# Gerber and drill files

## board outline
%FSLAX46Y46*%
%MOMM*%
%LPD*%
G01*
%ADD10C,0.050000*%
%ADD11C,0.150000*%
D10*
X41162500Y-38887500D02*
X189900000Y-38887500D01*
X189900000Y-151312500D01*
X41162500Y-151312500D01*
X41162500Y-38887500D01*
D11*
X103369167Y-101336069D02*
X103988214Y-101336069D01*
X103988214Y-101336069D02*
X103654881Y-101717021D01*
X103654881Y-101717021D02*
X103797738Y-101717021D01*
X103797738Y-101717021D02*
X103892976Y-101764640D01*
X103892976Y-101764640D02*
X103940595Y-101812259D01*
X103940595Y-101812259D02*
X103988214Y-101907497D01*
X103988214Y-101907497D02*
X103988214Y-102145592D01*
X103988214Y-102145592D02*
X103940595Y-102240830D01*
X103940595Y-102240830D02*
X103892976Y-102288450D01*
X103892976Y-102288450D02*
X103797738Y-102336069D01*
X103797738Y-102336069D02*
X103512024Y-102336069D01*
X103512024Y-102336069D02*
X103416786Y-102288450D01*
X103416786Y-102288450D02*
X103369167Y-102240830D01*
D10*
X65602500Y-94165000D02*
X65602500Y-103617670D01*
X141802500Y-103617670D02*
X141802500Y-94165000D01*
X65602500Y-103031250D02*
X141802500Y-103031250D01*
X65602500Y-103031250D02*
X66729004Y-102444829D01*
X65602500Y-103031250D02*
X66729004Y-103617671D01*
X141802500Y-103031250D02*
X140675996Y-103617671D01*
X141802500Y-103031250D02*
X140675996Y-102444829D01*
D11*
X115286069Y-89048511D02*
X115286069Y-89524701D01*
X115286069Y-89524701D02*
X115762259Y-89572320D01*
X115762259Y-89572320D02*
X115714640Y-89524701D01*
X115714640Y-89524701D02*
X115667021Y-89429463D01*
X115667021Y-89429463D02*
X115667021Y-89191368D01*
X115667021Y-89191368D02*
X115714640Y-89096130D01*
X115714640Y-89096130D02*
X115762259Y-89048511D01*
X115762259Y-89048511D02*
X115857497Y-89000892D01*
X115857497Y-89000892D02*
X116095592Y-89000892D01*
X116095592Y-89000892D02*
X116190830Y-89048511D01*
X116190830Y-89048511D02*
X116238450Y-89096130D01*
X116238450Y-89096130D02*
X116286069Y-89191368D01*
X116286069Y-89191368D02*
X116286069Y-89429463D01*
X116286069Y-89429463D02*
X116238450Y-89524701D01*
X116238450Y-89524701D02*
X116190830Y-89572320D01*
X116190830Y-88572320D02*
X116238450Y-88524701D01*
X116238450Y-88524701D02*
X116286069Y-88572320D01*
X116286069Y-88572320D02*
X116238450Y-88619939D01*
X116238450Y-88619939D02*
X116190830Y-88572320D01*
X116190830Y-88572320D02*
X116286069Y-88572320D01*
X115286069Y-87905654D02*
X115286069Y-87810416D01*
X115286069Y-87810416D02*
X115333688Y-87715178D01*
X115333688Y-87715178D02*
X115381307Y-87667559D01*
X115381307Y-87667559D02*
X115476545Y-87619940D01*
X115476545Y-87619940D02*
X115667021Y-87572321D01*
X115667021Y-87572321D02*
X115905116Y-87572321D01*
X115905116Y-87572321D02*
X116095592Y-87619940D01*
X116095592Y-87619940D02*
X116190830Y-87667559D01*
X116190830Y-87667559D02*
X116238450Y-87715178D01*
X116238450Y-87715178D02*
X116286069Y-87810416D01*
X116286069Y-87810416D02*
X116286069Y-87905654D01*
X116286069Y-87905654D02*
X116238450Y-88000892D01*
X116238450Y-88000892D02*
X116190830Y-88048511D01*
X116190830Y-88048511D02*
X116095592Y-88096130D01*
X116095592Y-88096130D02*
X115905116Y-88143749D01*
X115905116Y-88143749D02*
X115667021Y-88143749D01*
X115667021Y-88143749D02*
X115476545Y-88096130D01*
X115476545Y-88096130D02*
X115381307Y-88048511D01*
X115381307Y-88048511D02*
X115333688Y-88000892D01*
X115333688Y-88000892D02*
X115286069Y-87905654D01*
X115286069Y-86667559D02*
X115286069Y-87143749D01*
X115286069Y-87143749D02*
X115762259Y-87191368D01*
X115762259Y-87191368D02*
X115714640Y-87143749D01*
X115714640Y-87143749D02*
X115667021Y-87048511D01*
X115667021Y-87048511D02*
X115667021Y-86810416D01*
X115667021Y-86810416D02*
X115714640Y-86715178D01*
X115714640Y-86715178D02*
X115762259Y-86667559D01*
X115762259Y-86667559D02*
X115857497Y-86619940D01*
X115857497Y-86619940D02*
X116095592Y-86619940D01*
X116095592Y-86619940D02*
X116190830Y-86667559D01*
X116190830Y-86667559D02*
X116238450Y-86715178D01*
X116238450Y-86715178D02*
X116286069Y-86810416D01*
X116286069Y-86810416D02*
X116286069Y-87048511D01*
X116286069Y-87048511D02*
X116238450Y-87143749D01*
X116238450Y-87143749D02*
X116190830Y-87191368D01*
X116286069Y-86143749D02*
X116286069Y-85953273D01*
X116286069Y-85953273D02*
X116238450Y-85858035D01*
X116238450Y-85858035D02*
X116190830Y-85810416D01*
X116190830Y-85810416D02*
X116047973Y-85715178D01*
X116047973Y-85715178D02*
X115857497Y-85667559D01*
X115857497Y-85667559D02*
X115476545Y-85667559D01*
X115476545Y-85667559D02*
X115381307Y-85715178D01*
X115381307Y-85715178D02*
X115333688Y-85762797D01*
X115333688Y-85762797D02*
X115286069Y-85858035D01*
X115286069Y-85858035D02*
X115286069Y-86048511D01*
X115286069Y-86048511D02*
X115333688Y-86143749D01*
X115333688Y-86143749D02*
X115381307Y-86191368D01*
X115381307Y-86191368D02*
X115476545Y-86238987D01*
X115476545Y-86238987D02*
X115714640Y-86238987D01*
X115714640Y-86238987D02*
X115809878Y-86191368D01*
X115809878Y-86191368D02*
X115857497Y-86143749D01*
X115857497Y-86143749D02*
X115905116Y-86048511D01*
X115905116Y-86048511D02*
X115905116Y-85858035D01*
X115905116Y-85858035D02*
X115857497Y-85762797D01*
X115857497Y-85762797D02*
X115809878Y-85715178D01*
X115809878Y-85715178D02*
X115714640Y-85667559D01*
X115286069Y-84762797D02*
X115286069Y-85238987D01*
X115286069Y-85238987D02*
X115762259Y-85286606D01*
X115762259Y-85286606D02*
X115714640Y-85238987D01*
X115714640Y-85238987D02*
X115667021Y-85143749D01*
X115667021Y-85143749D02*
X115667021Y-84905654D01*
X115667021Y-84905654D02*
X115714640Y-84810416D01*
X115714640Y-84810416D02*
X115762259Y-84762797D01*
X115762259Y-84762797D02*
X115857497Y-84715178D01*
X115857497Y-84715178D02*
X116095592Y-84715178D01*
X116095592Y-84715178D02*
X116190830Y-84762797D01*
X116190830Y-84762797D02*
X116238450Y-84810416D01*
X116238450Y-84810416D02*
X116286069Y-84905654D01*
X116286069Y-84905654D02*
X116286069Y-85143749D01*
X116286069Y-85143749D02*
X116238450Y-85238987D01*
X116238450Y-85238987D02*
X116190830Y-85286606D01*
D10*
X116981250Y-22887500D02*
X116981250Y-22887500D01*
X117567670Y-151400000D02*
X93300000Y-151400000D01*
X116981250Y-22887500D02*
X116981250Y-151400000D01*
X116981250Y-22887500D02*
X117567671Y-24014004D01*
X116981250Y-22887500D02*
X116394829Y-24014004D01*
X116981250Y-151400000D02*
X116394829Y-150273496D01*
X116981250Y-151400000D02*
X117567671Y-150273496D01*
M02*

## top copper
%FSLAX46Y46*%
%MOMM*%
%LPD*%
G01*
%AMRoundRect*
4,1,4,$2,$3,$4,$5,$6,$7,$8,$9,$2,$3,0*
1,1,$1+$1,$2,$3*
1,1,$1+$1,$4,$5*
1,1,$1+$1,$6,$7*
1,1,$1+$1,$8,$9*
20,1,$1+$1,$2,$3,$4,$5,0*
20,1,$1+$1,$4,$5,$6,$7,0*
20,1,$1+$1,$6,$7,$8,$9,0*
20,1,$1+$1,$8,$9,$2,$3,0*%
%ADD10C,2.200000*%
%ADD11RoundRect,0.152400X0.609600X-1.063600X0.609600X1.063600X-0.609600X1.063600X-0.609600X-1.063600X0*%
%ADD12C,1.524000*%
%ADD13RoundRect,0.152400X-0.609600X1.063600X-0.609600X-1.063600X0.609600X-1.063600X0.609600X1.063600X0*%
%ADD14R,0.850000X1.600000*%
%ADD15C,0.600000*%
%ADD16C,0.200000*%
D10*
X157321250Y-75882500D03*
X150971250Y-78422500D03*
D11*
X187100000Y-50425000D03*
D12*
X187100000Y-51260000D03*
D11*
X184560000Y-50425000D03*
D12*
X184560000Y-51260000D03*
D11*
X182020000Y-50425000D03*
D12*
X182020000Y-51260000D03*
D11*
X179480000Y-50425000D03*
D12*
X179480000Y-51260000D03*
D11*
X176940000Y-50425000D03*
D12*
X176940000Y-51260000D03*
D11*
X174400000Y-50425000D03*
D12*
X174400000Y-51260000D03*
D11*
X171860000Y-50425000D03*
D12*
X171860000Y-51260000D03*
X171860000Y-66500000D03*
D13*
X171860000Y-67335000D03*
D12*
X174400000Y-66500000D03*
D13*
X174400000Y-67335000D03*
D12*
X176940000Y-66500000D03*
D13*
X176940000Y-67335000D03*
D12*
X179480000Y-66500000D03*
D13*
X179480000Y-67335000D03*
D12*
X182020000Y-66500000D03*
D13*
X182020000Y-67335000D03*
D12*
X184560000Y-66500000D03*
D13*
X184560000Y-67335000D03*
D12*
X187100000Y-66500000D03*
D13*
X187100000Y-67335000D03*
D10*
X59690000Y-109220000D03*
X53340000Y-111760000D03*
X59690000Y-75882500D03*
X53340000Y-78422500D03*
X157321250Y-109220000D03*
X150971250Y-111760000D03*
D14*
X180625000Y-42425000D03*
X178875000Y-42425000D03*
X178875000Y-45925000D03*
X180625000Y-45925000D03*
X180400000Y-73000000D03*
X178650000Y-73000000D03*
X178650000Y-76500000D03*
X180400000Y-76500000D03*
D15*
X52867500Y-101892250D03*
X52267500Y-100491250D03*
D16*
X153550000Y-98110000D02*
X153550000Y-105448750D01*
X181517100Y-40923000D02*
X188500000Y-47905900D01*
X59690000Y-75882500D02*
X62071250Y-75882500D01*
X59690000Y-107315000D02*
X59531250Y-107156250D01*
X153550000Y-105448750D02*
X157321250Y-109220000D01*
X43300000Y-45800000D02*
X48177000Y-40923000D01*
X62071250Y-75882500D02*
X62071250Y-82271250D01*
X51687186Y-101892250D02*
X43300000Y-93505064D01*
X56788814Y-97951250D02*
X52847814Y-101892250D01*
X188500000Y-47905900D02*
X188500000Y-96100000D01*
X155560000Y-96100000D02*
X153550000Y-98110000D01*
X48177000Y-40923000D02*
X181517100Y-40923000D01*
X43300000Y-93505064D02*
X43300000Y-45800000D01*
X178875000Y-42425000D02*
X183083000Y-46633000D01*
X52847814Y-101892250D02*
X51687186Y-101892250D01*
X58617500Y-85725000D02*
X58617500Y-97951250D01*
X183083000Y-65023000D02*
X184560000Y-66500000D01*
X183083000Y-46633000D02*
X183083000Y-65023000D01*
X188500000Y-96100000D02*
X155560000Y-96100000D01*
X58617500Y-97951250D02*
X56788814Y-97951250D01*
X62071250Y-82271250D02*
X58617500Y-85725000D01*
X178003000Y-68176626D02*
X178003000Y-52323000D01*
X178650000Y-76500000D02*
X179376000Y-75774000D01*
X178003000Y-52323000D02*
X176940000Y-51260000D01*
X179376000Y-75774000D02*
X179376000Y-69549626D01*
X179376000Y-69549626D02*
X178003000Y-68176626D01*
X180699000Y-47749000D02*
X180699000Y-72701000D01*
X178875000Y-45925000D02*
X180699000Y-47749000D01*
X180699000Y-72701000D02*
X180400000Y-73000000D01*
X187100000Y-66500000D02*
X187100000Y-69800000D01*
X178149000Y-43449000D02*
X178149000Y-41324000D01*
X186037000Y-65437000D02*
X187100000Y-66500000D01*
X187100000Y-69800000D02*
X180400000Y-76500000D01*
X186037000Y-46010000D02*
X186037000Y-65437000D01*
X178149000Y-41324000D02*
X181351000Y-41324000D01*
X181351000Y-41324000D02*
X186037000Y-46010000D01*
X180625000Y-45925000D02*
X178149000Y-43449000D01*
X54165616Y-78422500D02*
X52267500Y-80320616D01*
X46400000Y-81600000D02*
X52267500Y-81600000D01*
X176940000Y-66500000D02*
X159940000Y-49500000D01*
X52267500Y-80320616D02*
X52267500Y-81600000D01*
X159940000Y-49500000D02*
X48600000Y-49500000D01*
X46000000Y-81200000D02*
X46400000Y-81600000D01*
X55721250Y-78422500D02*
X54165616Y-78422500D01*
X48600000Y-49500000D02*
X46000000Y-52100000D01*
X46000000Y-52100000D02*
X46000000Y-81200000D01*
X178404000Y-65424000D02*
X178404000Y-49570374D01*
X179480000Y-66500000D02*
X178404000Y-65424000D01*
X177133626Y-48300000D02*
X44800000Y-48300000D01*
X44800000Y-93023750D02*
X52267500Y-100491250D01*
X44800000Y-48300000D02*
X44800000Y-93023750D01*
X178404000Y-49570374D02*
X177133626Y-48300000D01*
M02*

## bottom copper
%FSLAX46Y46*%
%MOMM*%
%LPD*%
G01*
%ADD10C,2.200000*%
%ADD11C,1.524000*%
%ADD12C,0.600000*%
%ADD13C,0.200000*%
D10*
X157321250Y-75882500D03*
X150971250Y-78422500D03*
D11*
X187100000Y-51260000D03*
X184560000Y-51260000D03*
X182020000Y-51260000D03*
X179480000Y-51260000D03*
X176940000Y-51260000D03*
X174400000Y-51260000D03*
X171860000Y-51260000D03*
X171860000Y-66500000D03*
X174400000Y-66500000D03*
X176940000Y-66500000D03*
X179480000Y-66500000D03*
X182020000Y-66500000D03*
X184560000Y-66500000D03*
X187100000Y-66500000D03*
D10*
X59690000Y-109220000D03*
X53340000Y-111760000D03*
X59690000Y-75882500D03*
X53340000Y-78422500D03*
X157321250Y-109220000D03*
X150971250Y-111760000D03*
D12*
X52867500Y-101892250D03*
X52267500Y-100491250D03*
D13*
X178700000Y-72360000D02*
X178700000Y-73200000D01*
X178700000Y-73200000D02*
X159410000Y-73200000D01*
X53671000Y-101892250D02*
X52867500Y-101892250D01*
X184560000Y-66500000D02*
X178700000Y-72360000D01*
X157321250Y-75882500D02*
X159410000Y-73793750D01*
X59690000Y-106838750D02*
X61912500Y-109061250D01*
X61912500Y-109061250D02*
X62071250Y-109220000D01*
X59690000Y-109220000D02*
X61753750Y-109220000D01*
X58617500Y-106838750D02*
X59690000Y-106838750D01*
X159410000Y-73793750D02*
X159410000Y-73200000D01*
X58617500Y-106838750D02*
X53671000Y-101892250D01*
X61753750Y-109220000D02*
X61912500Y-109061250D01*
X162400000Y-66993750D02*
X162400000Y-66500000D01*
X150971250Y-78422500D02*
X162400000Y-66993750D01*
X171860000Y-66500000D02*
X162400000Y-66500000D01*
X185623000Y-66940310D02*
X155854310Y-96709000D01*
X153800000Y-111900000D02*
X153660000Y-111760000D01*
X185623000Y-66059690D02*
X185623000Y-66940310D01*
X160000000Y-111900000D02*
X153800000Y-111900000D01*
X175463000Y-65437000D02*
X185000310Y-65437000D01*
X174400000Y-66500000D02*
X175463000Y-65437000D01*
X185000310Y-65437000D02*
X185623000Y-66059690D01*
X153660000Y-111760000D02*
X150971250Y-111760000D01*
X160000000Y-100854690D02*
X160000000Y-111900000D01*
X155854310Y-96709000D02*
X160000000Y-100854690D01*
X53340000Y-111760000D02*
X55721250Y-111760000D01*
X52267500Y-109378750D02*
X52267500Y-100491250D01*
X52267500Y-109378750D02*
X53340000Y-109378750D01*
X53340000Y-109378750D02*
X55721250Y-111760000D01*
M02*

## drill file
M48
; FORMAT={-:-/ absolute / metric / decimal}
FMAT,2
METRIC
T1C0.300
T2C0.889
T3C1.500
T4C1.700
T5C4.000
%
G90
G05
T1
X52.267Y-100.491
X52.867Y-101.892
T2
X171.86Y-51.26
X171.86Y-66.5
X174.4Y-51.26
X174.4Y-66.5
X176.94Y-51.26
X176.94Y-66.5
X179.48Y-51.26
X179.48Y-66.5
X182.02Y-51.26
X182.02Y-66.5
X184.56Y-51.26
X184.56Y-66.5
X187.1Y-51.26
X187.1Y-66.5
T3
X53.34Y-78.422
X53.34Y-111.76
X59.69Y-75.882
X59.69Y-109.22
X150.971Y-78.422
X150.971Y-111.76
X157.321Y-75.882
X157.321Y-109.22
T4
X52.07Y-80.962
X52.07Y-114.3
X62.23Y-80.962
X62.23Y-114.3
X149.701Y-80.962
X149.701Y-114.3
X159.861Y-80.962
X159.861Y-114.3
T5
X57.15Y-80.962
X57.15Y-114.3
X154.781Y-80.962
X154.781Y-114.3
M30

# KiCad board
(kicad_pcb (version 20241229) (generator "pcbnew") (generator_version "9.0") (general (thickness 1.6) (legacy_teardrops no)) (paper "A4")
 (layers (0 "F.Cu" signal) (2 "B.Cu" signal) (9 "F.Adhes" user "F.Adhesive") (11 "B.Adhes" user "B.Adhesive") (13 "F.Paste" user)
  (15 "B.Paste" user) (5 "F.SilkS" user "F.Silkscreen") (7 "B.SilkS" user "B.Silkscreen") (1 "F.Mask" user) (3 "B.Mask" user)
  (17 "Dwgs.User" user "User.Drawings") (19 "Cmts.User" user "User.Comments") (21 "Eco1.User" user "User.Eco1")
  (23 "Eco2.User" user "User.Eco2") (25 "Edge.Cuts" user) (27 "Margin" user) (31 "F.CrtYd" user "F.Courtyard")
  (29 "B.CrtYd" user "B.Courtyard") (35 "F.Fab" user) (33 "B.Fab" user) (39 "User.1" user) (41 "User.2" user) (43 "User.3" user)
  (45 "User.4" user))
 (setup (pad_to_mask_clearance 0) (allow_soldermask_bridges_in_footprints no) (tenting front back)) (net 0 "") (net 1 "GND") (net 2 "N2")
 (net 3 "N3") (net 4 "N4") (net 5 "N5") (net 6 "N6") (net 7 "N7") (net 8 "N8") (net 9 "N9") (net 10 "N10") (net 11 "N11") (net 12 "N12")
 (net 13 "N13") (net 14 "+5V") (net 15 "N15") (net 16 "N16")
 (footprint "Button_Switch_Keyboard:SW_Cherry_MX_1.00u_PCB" (layer "F.Cu") (at 157.32125 75.8825)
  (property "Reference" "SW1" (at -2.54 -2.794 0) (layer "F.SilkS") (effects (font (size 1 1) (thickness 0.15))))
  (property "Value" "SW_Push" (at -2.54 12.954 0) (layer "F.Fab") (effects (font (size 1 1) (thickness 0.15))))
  (pad "" np_thru_hole circle (at -7.62 5.08) (size 1.7 1.7) (drill 1.7) (layers "*.Cu" "*.Mask"))
  (pad "" np_thru_hole circle (at -2.54 5.08) (size 4 4) (drill 4) (layers "*.Cu" "*.Mask"))
  (pad "" np_thru_hole circle (at 2.54 5.08) (size 1.7 1.7) (drill 1.7) (layers "*.Cu" "*.Mask"))
  (pad "1" thru_hole circle (at 0 0) (size 2.2 2.2) (drill 1.5) (layers "*.Cu" "*.Mask") (remove_unused_layers no) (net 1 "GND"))
  (pad "2" thru_hole circle (at -6.35 2.54) (size 2.2 2.2) (drill 1.5) (layers "*.Cu" "*.Mask") (remove_unused_layers no) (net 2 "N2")))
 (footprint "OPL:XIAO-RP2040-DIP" (layer "F.Cu") (at 179.48 58.88 -90)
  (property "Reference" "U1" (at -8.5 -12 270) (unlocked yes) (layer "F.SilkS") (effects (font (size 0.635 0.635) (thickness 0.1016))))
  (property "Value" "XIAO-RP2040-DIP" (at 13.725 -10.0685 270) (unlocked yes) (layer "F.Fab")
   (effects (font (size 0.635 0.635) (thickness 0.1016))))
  (pad "1" smd roundrect (at -8.455 -7.62 90) (size 2.432 1.524) (layers "F.Cu" "F.Mask") (roundrect_rratio 0.1) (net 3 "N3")
   (thermal_bridge_angle 45))
  (pad "1" thru_hole circle (at -7.62 -7.62 90) (size 1.524 1.524) (drill 0.889) (layers "*.Cu" "*.Mask") (remove_unused_layers no)
   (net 3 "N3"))
  (pad "2" smd roundrect (at -8.455 -5.08 90) (size 2.432 1.524) (layers "F.Cu" "F.Mask") (roundrect_rratio 0.1) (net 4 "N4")
   (thermal_bridge_angle 45))
  (pad "2" thru_hole circle (at -7.62 -5.08 90) (size 1.524 1.524) (drill 0.889) (layers "*.Cu" "*.Mask") (remove_unused_layers no)
   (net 4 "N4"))
  (pad "3" smd roundrect (at -8.455 -2.54 90) (size 2.432 1.524) (layers "F.Cu" "F.Mask") (roundrect_rratio 0.1) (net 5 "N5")
   (thermal_bridge_angle 45))
  (pad "3" thru_hole circle (at -7.62 -2.54 90) (size 1.524 1.524) (drill 0.889) (layers "*.Cu" "*.Mask") (remove_unused_layers no)
   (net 5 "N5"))
  (pad "4" smd roundrect (at -8.455 0 90) (size 2.432 1.524) (layers "F.Cu" "F.Mask") (roundrect_rratio 0.1) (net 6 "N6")
   (thermal_bridge_angle 45))
  (pad "4" thru_hole circle (at -7.62 0 90) (size 1.524 1.524) (drill 0.889) (layers "*.Cu" "*.Mask") (remove_unused_layers no) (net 6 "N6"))
  (pad "5" smd roundrect (at -8.455 2.54 90) (size 2.432 1.524) (layers "F.Cu" "F.Mask") (roundrect_rratio 0.1) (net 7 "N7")
   (thermal_bridge_angle 45))
  (pad "5" thru_hole circle (at -7.62 2.54 90) (size 1.524 1.524) (drill 0.889) (layers "*.Cu" "*.Mask") (remove_unused_layers no)
   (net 7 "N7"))
  (pad "6" smd roundrect (at -8.455 5.08 90) (size 2.432 1.524) (layers "F.Cu" "F.Mask") (roundrect_rratio 0.1) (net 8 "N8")
   (thermal_bridge_angle 45))
  (pad "6" thru_hole circle (at -7.62 5.08 90) (size 1.524 1.524) (drill 0.889) (layers "*.Cu" "*.Mask") (remove_unused_layers no)
   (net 8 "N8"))
  (pad "7" smd roundrect (at -8.455 7.62 90) (size 2.432 1.524) (layers "F.Cu" "F.Mask") (roundrect_rratio 0.1) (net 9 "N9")
   (thermal_bridge_angle 45))
  (pad "7" thru_hole circle (at -7.62 7.62 90) (size 1.524 1.524) (drill 0.889) (layers "*.Cu" "*.Mask") (remove_unused_layers no)
   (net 9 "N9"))
  (pad "8" thru_hole circle (at 7.62 7.62 270) (size 1.524 1.524) (drill 0.889) (layers "*.Cu" "*.Mask") (remove_unused_layers no)
   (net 2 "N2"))
  (pad "8" smd roundrect (at 8.455 7.62 270) (size 2.432 1.524) (layers "F.Cu" "F.Mask") (roundrect_rratio 0.1) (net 2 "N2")
   (thermal_bridge_angle 45))
  (pad "9" thru_hole circle (at 7.62 5.08 270) (size 1.524 1.524) (drill 0.889) (layers "*.Cu" "*.Mask") (remove_unused_layers no)
   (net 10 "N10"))
  (pad "9" smd roundrect (at 8.455 5.08 270) (size 2.432 1.524) (layers "F.Cu" "F.Mask") (roundrect_rratio 0.1) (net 10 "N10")
   (thermal_bridge_angle 45))
  (pad "10" thru_hole circle (at 7.62 2.54 270) (size 1.524 1.524) (drill 0.889) (layers "*.Cu" "*.Mask") (remove_unused_layers no)
   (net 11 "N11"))
  (pad "10" smd roundrect (at 8.455 2.54 270) (size 2.432 1.524) (layers "F.Cu" "F.Mask") (roundrect_rratio 0.1) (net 11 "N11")
   (thermal_bridge_angle 45))
  (pad "11" thru_hole circle (at 7.62 0 270) (size 1.524 1.524) (drill 0.889) (layers "*.Cu" "*.Mask") (remove_unused_layers no)
   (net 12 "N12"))
  (pad "11" smd roundrect (at 8.455 0 270) (size 2.432 1.524) (layers "F.Cu" "F.Mask") (roundrect_rratio 0.1) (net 12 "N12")
   (thermal_bridge_angle 45))
  (pad "12" thru_hole circle (at 7.62 -2.54 270) (size 1.524 1.524) (drill 0.889) (layers "*.Cu" "*.Mask") (remove_unused_layers no)
   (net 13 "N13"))
  (pad "12" smd roundrect (at 8.455 -2.54 270) (size 2.432 1.524) (layers "F.Cu" "F.Mask") (roundrect_rratio 0.1) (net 13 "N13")
   (thermal_bridge_angle 45))
  (pad "13" thru_hole circle (at 7.62 -5.08 270) (size 1.524 1.524) (drill 0.889) (layers "*.Cu" "*.Mask") (remove_unused_layers no)
   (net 1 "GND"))
  (pad "13" smd roundrect (at 8.455 -5.08 270) (size 2.432 1.524) (layers "F.Cu" "F.Mask") (roundrect_rratio 0.1) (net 1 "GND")
   (thermal_bridge_angle 45))
  (pad "14" thru_hole circle (at 7.62 -7.62 270) (size 1.524 1.524) (drill 0.889) (layers "*.Cu" "*.Mask") (remove_unused_layers no)
   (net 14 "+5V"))
  (pad "14" smd roundrect (at 8.455 -7.62 270) (size 2.432 1.524) (layers "F.Cu" "F.Mask") (roundrect_rratio 0.1) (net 14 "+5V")
   (thermal_bridge_angle 45)))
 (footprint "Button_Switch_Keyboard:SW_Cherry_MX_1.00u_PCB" (layer "F.Cu") (at 59.69 109.22)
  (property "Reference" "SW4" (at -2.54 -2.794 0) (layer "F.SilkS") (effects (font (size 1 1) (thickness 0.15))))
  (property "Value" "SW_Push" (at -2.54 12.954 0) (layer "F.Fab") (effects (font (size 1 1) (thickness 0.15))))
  (pad "" np_thru_hole circle (at -7.62 5.08) (size 1.7 1.7) (drill 1.7) (layers "*.Cu" "*.Mask"))
  (pad "" np_thru_hole circle (at -2.54 5.08) (size 4 4) (drill 4) (layers "*.Cu" "*.Mask"))
  (pad "" np_thru_hole circle (at 2.54 5.08) (size 1.7 1.7) (drill 1.7) (layers "*.Cu" "*.Mask"))
  (pad "1" thru_hole circle (at 0 0) (size 2.2 2.2) (drill 1.5) (layers "*.Cu" "*.Mask") (remove_unused_layers no) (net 1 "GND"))
  (pad "2" thru_hole circle (at -6.35 2.54) (size 2.2 2.2) (drill 1.5) (layers "*.Cu" "*.Mask") (remove_unused_layers no) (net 12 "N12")))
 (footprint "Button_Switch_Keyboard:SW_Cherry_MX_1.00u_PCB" (layer "F.Cu") (at 59.69 75.8825)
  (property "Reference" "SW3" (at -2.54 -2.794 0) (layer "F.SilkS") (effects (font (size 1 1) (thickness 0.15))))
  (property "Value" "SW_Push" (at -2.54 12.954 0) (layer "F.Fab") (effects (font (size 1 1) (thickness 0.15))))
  (pad "" np_thru_hole circle (at -7.62 5.08) (size 1.7 1.7) (drill 1.7) (layers "*.Cu" "*.Mask"))
  (pad "" np_thru_hole circle (at -2.54 5.08) (size 4 4) (drill 4) (layers "*.Cu" "*.Mask"))
  (pad "" np_thru_hole circle (at 2.54 5.08) (size 1.7 1.7) (drill 1.7) (layers "*.Cu" "*.Mask"))
  (pad "1" thru_hole circle (at 0 0) (size 2.2 2.2) (drill 1.5) (layers "*.Cu" "*.Mask") (remove_unused_layers no) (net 1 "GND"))
  (pad "2" thru_hole circle (at -6.35 2.54) (size 2.2 2.2) (drill 1.5) (layers "*.Cu" "*.Mask") (remove_unused_layers no) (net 11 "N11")))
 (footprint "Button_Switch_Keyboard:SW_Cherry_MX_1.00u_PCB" (layer "F.Cu") (at 157.32125 109.22)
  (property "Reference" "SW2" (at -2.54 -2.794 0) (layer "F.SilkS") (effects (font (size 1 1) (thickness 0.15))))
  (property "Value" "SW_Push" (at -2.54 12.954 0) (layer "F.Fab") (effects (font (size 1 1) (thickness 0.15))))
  (pad "" np_thru_hole circle (at -7.62 5.08) (size 1.7 1.7) (drill 1.7) (layers "*.Cu" "*.Mask"))
  (pad "" np_thru_hole circle (at -2.54 5.08) (size 4 4) (drill 4) (layers "*.Cu" "*.Mask"))
  (pad "" np_thru_hole circle (at 2.54 5.08) (size 1.7 1.7) (drill 1.7) (layers "*.Cu" "*.Mask"))
  (pad "1" thru_hole circle (at 0 0) (size 2.2 2.2) (drill 1.5) (layers "*.Cu" "*.Mask") (remove_unused_layers no) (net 1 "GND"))
  (pad "2" thru_hole circle (at -6.35 2.54) (size 2.2 2.2) (drill 1.5) (layers "*.Cu" "*.Mask") (remove_unused_layers no) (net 10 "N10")))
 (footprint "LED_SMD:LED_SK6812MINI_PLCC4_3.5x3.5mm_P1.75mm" (layer "F.Cu") (at 179.75 44.175 -90)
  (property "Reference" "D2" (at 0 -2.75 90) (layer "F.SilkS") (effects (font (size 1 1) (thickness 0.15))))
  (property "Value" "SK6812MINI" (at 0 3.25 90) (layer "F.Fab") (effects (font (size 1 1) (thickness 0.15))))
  (pad "1" smd rect (at -1.75 -0.875 270) (size 1.6 0.85) (layers "F.Cu" "F.Mask" "F.Paste") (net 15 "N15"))
  (pad "2" smd rect (at -1.75 0.875 270) (size 1.6 0.85) (layers "F.Cu" "F.Mask" "F.Paste") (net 1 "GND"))
  (pad "3" smd rect (at 1.75 0.875 270) (size 1.6 0.85) (layers "F.Cu" "F.Mask" "F.Paste") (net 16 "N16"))
  (pad "4" smd rect (at 1.75 -0.875 270) (size 1.6 0.85) (layers "F.Cu" "F.Mask" "F.Paste") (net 14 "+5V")))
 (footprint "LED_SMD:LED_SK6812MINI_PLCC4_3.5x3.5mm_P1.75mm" (layer "F.Cu") (at 179.525 74.75 -90)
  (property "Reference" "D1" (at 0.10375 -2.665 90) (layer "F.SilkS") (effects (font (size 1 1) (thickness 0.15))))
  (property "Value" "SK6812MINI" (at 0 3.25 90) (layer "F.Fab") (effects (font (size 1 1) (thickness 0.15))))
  (pad "1" smd rect (at -1.75 -0.875 270) (size 1.6 0.85) (layers "F.Cu" "F.Mask" "F.Paste") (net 16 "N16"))
  (pad "2" smd rect (at -1.75 0.875 270) (size 1.6 0.85) (layers "F.Cu" "F.Mask" "F.Paste") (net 1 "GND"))
  (pad "3" smd rect (at 1.75 0.875 270) (size 1.6 0.85) (layers "F.Cu" "F.Mask" "F.Paste") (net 7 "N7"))
  (pad "4" smd rect (at 1.75 -0.875 270) (size 1.6 0.85) (layers "F.Cu" "F.Mask" "F.Paste") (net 14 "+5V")))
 (gr_rect (start 41.1625 38.8875) (end 189.9 151.3125) (stroke (width 0.05) (type solid)) (fill no) (layer "Edge.Cuts"))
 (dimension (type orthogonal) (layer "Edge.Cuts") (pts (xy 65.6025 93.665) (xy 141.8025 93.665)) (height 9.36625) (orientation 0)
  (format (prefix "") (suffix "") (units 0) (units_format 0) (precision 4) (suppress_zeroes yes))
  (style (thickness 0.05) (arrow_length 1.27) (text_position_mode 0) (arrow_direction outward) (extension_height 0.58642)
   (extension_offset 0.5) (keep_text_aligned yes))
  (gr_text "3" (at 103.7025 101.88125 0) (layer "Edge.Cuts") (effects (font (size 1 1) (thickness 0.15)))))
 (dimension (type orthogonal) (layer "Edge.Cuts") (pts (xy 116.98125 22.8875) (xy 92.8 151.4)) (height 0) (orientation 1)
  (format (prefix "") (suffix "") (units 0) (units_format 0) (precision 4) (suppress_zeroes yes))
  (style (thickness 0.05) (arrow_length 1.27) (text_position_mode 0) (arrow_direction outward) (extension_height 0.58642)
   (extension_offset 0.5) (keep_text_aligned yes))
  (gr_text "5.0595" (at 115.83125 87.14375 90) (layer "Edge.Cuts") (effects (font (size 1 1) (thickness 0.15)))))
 (segment (start 153.55 98.11) (end 153.55 105.44875) (width 0.2) (layer "F.Cu") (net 1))
 (segment (start 181.5171 40.923) (end 188.5 47.9059) (width 0.2) (layer "F.Cu") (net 1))
 (segment (start 59.69 75.8825) (end 62.07125 75.8825) (width 0.2) (layer "F.Cu") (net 1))
 (segment (start 59.69 107.315) (end 59.53125 107.15625) (width 0.2) (layer "F.Cu") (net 1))
 (segment (start 153.55 105.44875) (end 157.32125 109.22) (width 0.2) (layer "F.Cu") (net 1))
 (segment (start 43.3 45.8) (end 48.177 40.923) (width 0.2) (layer "F.Cu") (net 1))
 (segment (start 62.07125 75.8825) (end 62.07125 82.27125) (width 0.2) (layer "F.Cu") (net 1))
 (segment (start 51.687186 101.89225) (end 43.3 93.505064) (width 0.2) (layer "F.Cu") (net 1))
 (segment (start 56.788814 97.95125) (end 52.847814 101.89225) (width 0.2) (layer "F.Cu") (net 1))
 (segment (start 188.5 47.9059) (end 188.5 96.1) (width 0.2) (layer "F.Cu") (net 1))
 (segment (start 155.56 96.1) (end 153.55 98.11) (width 0.2) (layer "F.Cu") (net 1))
 (segment (start 48.177 40.923) (end 181.5171 40.923) (width 0.2) (layer "F.Cu") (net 1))
 (segment (start 43.3 93.505064) (end 43.3 45.8) (width 0.2) (layer "F.Cu") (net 1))
 (segment (start 178.875 42.425) (end 183.083 46.633) (width 0.2) (layer "F.Cu") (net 1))
 (segment (start 52.847814 101.89225) (end 51.687186 101.89225) (width 0.2) (layer "F.Cu") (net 1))
 (segment (start 58.6175 85.725) (end 58.6175 97.95125) (width 0.2) (layer "F.Cu") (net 1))
 (segment (start 183.083 65.023) (end 184.56 66.5) (width 0.2) (layer "F.Cu") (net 1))
 (segment (start 183.083 46.633) (end 183.083 65.023) (width 0.2) (layer "F.Cu") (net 1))
 (segment (start 188.5 96.1) (end 155.56 96.1) (width 0.2) (layer "F.Cu") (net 1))
 (segment (start 58.6175 97.95125) (end 56.788814 97.95125) (width 0.2) (layer "F.Cu") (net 1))
 (segment (start 62.07125 82.27125) (end 58.6175 85.725) (width 0.2) (layer "F.Cu") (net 1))
 (via (at 52.8675 101.89225) (size 0.6) (drill 0.3) (layers "F.Cu" "B.Cu") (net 1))
 (segment (start 178.7 72.36) (end 178.7 73.2) (width 0.2) (layer "B.Cu") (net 1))
 (segment (start 178.7 73.2) (end 159.41 73.2) (width 0.2) (layer "B.Cu") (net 1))
 (segment (start 53.671 101.89225) (end 52.8675 101.89225) (width 0.2) (layer "B.Cu") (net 1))
 (segment (start 184.56 66.5) (end 178.7 72.36) (width 0.2) (layer "B.Cu") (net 1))
 (segment (start 157.32125 75.8825) (end 159.41 73.79375) (width 0.2) (layer "B.Cu") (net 1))
 (segment (start 59.69 106.83875) (end 61.9125 109.06125) (width 0.2) (layer "B.Cu") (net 1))
 (segment (start 61.9125 109.06125) (end 62.07125 109.22) (width 0.2) (layer "B.Cu") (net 1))
 (segment (start 59.69 109.22) (end 61.75375 109.22) (width 0.2) (layer "B.Cu") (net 1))
 (segment (start 58.6175 106.83875) (end 59.69 106.83875) (width 0.2) (layer "B.Cu") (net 1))
 (segment (start 159.41 73.79375) (end 159.41 73.2) (width 0.2) (layer "B.Cu") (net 1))
 (segment (start 58.6175 106.83875) (end 53.671 101.89225) (width 0.2) (layer "B.Cu") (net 1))
 (segment (start 61.75375 109.22) (end 61.9125 109.06125) (width 0.2) (layer "B.Cu") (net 1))
 (segment (start 178.003 68.176626) (end 178.003 52.323) (width 0.2) (layer "F.Cu") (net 7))
 (segment (start 178.65 76.5) (end 179.376 75.774) (width 0.2) (layer "F.Cu") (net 7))
 (segment (start 178.003 52.323) (end 176.94 51.26) (width 0.2) (layer "F.Cu") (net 7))
 (segment (start 179.376 75.774) (end 179.376 69.549626) (width 0.2) (layer "F.Cu") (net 7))
 (segment (start 179.376 69.549626) (end 178.003 68.176626) (width 0.2) (layer "F.Cu") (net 7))
 (segment (start 180.699 47.749) (end 180.699 72.701) (width 0.2) (layer "F.Cu") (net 16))
 (segment (start 178.875 45.925) (end 180.699 47.749) (width 0.2) (layer "F.Cu") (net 16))
 (segment (start 180.699 72.701) (end 180.4 73) (width 0.2) (layer "F.Cu") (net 16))
 (segment (start 187.1 66.5) (end 187.1 69.8) (width 0.2) (layer "F.Cu") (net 14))
 (segment (start 178.149 43.449) (end 178.149 41.324) (width 0.2) (layer "F.Cu") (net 14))
 (segment (start 186.037 65.437) (end 187.1 66.5) (width 0.2) (layer "F.Cu") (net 14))
 (segment (start 187.1 69.8) (end 180.4 76.5) (width 0.2) (layer "F.Cu") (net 14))
 (segment (start 186.037 46.01) (end 186.037 65.437) (width 0.2) (layer "F.Cu") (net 14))
 (segment (start 178.149 41.324) (end 181.351 41.324) (width 0.2) (layer "F.Cu") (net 14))
 (segment (start 181.351 41.324) (end 186.037 46.01) (width 0.2) (layer "F.Cu") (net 14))
 (segment (start 180.625 45.925) (end 178.149 43.449) (width 0.2) (layer "F.Cu") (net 14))
 (segment (start 162.4 66.99375) (end 162.4 66.5) (width 0.2) (layer "B.Cu") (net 2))
 (segment (start 150.97125 78.4225) (end 162.4 66.99375) (width 0.2) (layer "B.Cu") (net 2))
 (segment (start 171.86 66.5) (end 162.4 66.5) (width 0.2) (layer "B.Cu") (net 2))
 (segment (start 185.623 66.94031) (end 155.85431 96.709) (width 0.2) (layer "B.Cu") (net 10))
 (segment (start 153.8 111.9) (end 153.66 111.76) (width 0.2) (layer "B.Cu") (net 10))
 (segment (start 185.623 66.05969) (end 185.623 66.94031) (width 0.2) (layer "B.Cu") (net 10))
 (segment (start 160 111.9) (end 153.8 111.9) (width 0.2) (layer "B.Cu") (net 10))
 (segment (start 175.463 65.437) (end 185.00031 65.437) (width 0.2) (layer "B.Cu") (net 10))
 (segment (start 174.4 66.5) (end 175.463 65.437) (width 0.2) (layer "B.Cu") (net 10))
 (segment (start 185.00031 65.437) (end 185.623 66.05969) (width 0.2) (layer "B.Cu") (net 10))
 (segment (start 153.66 111.76) (end 150.97125 111.76) (width 0.2) (layer "B.Cu") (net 10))
 (segment (start 160 100.85469) (end 160 111.9) (width 0.2) (layer "B.Cu") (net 10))
 (segment (start 155.85431 96.709) (end 160 100.85469) (width 0.2) (layer "B.Cu") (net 10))
 (segment (start 54.165616 78.4225) (end 52.2675 80.320616) (width 0.2) (layer "F.Cu") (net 11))
 (segment (start 46.4 81.6) (end 52.2675 81.6) (width 0.2) (layer "F.Cu") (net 11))
 (segment (start 176.94 66.5) (end 159.94 49.5) (width 0.2) (layer "F.Cu") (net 11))
 (segment (start 52.2675 80.320616) (end 52.2675 81.6) (width 0.2) (layer "F.Cu") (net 11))
 (segment (start 159.94 49.5) (end 48.6 49.5) (width 0.2) (layer "F.Cu") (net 11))
 (segment (start 46 81.2) (end 46.4 81.6) (width 0.2) (layer "F.Cu") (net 11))
 (segment (start 55.72125 78.4225) (end 54.165616 78.4225) (width 0.2) (layer "F.Cu") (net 11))
 (segment (start 48.6 49.5) (end 46 52.1) (width 0.2) (layer "F.Cu") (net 11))
 (segment (start 46 52.1) (end 46 81.2) (width 0.2) (layer "F.Cu") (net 11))
 (segment (start 178.404 65.424) (end 178.404 49.570374) (width 0.2) (layer "F.Cu") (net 12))
 (segment (start 179.48 66.5) (end 178.404 65.424) (width 0.2) (layer "F.Cu") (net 12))
 (segment (start 177.133626 48.3) (end 44.8 48.3) (width 0.2) (layer "F.Cu") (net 12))
 (segment (start 44.8 93.02375) (end 52.2675 100.49125) (width 0.2) (layer "F.Cu") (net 12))
 (segment (start 44.8 48.3) (end 44.8 93.02375) (width 0.2) (layer "F.Cu") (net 12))
 (segment (start 178.404 49.570374) (end 177.133626 48.3) (width 0.2) (layer "F.Cu") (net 12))
 (via (at 52.2675 100.49125) (size 0.6) (drill 0.3) (layers "F.Cu" "B.Cu") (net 12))
 (segment (start 53.34 111.76) (end 55.72125 111.76) (width 0.2) (layer "B.Cu") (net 12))
 (segment (start 52.2675 109.37875) (end 52.2675 100.49125) (width 0.2) (layer "B.Cu") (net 12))
 (segment (start 52.2675 109.37875) (end 53.34 109.37875) (width 0.2) (layer "B.Cu") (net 12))
 (segment (start 53.34 109.37875) (end 55.72125 111.76) (width 0.2) (layer "B.Cu") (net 12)))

